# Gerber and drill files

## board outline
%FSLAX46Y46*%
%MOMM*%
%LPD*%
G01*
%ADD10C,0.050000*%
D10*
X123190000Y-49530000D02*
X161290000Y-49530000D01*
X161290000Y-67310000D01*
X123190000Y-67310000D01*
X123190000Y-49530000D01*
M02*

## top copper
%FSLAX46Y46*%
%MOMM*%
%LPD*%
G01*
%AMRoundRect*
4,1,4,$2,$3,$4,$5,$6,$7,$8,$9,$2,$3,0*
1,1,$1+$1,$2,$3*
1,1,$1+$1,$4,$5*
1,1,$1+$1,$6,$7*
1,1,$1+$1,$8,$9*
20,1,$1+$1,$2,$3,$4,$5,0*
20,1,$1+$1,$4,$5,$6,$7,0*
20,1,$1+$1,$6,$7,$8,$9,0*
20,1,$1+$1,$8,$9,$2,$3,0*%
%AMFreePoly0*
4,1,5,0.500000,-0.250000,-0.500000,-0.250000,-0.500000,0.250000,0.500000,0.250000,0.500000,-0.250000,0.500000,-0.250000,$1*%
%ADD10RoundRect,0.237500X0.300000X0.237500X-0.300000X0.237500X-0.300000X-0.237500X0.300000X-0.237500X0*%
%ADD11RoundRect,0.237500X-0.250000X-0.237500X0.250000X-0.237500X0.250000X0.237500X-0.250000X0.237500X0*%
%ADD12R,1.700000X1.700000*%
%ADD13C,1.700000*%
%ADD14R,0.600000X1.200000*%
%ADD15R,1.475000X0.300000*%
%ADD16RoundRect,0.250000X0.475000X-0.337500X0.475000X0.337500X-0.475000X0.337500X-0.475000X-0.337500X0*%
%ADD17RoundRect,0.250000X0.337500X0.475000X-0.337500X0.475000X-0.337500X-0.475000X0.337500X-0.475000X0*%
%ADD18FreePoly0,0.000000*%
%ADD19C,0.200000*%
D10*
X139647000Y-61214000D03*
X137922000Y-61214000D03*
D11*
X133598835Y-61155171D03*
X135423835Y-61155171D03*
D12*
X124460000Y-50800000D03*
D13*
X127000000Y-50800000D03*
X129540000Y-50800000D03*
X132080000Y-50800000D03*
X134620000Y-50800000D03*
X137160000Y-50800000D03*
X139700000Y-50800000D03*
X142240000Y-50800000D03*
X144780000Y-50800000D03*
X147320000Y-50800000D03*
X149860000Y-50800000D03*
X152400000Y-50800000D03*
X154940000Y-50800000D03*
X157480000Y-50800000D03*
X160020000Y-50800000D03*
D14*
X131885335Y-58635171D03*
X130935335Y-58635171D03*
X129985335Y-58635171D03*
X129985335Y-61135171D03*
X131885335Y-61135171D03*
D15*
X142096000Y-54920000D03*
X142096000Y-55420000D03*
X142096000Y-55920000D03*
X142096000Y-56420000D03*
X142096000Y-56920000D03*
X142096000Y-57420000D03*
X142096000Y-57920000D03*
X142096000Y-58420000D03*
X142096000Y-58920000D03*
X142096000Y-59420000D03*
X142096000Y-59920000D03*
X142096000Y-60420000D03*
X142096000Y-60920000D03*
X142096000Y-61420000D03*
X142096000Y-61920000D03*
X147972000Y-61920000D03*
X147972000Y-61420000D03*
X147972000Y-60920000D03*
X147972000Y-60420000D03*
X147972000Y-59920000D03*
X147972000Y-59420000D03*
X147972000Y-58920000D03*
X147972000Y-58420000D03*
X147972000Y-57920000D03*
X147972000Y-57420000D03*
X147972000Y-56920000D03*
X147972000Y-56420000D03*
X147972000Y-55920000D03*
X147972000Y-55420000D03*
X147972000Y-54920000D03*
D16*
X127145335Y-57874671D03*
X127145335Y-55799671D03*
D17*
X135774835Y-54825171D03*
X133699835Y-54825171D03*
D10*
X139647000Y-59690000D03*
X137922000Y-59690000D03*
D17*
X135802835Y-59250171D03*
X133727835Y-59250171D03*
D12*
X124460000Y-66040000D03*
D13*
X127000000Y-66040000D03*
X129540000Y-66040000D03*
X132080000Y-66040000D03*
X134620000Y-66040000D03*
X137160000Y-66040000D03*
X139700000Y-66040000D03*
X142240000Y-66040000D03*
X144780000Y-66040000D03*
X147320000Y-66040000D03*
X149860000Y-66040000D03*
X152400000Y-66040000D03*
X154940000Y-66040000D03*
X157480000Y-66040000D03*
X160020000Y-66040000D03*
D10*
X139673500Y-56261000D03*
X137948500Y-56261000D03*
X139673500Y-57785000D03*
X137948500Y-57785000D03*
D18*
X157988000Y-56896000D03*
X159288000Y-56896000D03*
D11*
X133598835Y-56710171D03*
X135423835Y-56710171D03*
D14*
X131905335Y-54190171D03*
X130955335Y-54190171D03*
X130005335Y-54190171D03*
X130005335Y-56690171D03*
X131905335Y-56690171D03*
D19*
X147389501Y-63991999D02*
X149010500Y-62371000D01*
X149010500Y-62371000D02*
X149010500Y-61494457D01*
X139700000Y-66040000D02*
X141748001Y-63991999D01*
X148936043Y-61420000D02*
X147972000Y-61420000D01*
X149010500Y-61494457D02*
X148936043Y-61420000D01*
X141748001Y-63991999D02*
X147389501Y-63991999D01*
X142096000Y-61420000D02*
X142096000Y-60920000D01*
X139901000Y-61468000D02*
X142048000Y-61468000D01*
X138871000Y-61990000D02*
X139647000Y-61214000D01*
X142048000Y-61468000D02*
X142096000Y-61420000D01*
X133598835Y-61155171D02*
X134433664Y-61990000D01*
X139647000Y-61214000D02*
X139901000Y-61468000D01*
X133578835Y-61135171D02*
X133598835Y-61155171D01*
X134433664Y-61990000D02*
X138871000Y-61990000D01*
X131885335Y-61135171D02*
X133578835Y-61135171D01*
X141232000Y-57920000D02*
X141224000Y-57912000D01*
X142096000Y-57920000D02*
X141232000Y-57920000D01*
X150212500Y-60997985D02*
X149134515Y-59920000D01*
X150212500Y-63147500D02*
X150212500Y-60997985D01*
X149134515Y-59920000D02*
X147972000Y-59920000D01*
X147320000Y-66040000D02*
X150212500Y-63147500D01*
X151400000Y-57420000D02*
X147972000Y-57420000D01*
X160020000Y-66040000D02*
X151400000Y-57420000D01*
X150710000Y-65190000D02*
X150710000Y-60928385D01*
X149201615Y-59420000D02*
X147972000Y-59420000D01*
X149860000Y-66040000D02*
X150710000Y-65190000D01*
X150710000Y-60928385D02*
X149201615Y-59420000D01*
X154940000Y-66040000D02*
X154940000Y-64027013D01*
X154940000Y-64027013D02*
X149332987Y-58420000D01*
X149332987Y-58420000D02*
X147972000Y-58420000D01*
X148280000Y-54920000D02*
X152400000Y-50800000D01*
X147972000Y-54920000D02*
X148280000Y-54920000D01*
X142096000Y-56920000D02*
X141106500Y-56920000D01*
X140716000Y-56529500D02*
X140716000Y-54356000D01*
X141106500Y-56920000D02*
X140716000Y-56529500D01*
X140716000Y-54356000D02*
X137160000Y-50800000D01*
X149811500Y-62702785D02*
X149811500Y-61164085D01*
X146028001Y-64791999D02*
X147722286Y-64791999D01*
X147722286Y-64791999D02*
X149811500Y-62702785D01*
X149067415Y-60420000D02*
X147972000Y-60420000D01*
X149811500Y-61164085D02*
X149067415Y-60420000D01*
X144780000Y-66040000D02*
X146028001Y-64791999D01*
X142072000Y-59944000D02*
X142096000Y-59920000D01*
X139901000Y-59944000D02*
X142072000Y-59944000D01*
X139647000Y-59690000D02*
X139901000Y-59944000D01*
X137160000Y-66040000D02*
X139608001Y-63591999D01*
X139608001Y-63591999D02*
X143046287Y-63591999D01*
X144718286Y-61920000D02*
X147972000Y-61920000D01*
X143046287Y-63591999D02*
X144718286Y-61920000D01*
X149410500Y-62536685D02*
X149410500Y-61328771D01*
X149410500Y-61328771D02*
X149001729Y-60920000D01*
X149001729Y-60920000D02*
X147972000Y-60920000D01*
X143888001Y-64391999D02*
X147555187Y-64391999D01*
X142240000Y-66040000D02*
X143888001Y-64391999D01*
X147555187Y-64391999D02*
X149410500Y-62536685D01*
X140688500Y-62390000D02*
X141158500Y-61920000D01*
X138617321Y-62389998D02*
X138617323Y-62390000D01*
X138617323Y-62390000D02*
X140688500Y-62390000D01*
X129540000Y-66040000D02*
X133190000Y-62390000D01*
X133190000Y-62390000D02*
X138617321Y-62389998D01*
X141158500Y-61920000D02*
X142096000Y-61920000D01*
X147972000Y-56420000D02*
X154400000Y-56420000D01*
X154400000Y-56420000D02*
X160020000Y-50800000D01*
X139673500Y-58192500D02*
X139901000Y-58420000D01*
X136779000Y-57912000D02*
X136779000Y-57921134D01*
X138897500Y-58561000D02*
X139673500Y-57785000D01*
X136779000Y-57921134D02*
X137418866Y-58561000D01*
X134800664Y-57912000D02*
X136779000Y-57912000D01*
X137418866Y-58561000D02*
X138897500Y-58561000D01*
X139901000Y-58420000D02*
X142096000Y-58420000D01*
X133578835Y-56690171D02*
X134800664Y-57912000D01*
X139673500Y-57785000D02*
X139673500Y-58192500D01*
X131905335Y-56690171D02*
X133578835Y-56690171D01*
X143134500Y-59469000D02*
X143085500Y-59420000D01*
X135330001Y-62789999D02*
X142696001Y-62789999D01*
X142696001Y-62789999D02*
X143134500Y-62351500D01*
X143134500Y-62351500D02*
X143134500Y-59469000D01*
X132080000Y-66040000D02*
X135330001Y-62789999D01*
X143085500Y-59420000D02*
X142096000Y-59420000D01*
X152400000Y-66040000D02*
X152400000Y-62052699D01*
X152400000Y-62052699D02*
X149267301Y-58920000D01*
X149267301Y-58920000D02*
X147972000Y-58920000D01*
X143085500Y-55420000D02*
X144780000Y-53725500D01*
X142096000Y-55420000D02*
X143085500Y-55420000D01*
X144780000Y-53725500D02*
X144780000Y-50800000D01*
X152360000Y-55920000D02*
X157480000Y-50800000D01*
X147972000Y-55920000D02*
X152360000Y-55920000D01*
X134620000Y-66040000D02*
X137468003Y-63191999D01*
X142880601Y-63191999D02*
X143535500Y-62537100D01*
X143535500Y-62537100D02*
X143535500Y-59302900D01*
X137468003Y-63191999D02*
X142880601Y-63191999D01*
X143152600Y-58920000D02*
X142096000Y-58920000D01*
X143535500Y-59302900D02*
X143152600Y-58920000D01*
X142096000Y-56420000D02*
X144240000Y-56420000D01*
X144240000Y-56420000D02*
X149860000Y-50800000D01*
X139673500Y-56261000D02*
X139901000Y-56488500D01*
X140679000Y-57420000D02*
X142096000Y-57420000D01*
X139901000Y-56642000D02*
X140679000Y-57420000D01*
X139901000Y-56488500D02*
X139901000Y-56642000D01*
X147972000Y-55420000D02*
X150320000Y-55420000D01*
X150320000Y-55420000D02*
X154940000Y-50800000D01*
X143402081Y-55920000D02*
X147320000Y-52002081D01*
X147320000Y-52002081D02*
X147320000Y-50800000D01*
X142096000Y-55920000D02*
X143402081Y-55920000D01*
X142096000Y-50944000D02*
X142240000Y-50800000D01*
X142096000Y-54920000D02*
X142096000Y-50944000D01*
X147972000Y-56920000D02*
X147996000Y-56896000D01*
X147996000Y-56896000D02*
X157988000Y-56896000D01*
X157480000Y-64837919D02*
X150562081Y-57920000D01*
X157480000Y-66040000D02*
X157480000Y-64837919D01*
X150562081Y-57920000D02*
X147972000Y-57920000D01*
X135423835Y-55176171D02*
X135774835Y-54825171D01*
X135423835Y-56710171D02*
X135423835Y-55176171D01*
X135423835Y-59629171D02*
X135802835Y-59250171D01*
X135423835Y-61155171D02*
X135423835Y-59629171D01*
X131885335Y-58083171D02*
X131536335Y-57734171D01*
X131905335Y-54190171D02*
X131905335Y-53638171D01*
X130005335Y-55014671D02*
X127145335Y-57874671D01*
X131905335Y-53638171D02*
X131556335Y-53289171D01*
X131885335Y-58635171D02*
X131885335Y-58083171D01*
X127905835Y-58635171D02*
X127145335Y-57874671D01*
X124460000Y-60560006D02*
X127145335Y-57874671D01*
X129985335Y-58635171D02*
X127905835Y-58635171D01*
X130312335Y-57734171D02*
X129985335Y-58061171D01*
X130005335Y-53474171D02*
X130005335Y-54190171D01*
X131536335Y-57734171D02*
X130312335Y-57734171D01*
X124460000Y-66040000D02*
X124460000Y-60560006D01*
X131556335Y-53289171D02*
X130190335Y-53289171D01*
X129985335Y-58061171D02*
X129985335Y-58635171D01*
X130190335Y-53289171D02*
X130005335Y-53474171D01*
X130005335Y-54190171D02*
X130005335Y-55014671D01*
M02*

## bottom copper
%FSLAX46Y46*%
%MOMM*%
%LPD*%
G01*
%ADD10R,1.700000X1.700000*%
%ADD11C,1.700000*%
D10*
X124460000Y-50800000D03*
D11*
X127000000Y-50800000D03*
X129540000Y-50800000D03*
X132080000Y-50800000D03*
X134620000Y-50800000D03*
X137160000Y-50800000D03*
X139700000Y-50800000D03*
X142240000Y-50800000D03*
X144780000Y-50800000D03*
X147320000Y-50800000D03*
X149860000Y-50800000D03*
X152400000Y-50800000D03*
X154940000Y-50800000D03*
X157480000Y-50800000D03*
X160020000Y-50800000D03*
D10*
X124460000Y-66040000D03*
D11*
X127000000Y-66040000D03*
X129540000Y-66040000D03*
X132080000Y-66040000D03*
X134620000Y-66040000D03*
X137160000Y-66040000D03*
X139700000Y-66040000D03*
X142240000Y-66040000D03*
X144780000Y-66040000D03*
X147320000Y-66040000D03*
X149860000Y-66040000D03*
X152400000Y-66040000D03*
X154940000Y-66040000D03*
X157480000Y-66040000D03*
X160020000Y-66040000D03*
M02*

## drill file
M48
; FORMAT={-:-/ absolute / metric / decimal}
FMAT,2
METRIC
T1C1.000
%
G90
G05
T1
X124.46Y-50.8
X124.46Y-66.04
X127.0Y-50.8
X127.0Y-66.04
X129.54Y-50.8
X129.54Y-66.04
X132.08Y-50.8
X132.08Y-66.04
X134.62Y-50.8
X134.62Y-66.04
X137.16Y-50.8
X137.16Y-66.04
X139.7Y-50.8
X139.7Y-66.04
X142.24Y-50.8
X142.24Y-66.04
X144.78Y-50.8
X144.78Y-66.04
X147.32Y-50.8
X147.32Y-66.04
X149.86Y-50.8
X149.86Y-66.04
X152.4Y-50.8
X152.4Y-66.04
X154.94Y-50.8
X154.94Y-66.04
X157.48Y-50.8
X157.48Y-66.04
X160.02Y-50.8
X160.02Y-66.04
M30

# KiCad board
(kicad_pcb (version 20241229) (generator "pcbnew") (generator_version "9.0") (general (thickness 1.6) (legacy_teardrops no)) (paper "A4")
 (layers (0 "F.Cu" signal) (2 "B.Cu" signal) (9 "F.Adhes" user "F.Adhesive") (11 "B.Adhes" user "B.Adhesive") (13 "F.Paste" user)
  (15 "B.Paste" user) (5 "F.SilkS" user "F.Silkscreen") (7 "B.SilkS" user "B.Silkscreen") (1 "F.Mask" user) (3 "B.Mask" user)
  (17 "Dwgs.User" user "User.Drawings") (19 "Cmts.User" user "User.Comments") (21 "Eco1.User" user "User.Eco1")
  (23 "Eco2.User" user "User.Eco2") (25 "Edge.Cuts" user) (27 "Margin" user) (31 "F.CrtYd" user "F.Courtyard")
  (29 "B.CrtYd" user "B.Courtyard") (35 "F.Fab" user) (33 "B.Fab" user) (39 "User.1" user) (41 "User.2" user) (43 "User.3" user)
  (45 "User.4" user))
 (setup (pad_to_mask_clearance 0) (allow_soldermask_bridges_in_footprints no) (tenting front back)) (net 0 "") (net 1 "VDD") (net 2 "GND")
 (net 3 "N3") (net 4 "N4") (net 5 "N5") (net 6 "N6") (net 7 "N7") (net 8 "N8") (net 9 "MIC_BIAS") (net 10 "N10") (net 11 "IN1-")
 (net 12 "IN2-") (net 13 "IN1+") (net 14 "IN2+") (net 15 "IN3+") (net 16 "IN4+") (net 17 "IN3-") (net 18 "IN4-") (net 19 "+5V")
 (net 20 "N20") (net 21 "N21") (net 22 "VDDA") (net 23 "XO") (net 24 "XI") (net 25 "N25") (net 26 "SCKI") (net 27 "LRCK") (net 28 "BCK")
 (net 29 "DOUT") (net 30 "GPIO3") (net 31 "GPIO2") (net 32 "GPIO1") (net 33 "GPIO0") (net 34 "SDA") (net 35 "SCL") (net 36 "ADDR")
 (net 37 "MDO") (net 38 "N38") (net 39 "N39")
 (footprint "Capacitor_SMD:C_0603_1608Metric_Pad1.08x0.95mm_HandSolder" (layer "F.Cu") (at 138.7845 61.214 180)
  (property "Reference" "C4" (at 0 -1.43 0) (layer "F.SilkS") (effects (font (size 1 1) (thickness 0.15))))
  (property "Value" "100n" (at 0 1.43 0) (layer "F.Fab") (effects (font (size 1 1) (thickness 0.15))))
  (pad "1" smd roundrect (at -0.8625 0 180) (size 1.075 0.95) (layers "F.Cu" "F.Mask" "F.Paste") (roundrect_rratio 0.25) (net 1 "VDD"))
  (pad "2" smd roundrect (at 0.8625 0 180) (size 1.075 0.95) (layers "F.Cu" "F.Mask" "F.Paste") (roundrect_rratio 0.25) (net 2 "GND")))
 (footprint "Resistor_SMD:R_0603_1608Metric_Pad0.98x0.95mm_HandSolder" (layer "F.Cu") (at 134.511335 61.155171)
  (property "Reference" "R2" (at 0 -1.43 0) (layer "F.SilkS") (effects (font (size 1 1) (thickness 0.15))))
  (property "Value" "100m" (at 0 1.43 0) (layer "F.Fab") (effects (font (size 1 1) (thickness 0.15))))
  (pad "1" smd roundrect (at -0.9125 0) (size 0.975 0.95) (layers "F.Cu" "F.Mask" "F.Paste") (roundrect_rratio 0.25) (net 1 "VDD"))
  (pad "2" smd roundrect (at 0.9125 0) (size 0.975 0.95) (layers "F.Cu" "F.Mask" "F.Paste") (roundrect_rratio 0.25) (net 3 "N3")))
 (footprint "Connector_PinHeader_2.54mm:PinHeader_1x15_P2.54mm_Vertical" (layer "F.Cu") (at 124.46 50.8 90)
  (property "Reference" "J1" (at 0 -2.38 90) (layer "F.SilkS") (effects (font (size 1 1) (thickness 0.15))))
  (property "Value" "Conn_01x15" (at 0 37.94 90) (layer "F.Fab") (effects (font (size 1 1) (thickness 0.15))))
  (pad "1" thru_hole rect (at 0 0 90) (size 1.7 1.7) (drill 1) (layers "*.Cu" "*.Mask") (remove_unused_layers no) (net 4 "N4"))
  (pad "2" thru_hole circle (at 0 2.54 90) (size 1.7 1.7) (drill 1) (layers "*.Cu" "*.Mask") (remove_unused_layers no) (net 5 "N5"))
  (pad "3" thru_hole circle (at 0 5.08 90) (size 1.7 1.7) (drill 1) (layers "*.Cu" "*.Mask") (remove_unused_layers no) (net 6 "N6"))
  (pad "4" thru_hole circle (at 0 7.62 90) (size 1.7 1.7) (drill 1) (layers "*.Cu" "*.Mask") (remove_unused_layers no) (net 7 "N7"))
  (pad "5" thru_hole circle (at 0 10.16 90) (size 1.7 1.7) (drill 1) (layers "*.Cu" "*.Mask") (remove_unused_layers no) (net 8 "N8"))
  (pad "6" thru_hole circle (at 0 12.7 90) (size 1.7 1.7) (drill 1) (layers "*.Cu" "*.Mask") (remove_unused_layers no) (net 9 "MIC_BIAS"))
  (pad "7" thru_hole circle (at 0 15.24 90) (size 1.7 1.7) (drill 1) (layers "*.Cu" "*.Mask") (remove_unused_layers no) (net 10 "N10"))
  (pad "8" thru_hole circle (at 0 17.78 90) (size 1.7 1.7) (drill 1) (layers "*.Cu" "*.Mask") (remove_unused_layers no) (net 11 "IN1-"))
  (pad "9" thru_hole circle (at 0 20.32 90) (size 1.7 1.7) (drill 1) (layers "*.Cu" "*.Mask") (remove_unused_layers no) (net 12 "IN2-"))
  (pad "10" thru_hole circle (at 0 22.86 90) (size 1.7 1.7) (drill 1) (layers "*.Cu" "*.Mask") (remove_unused_layers no) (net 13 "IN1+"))
  (pad "11" thru_hole circle (at 0 25.4 90) (size 1.7 1.7) (drill 1) (layers "*.Cu" "*.Mask") (remove_unused_layers no) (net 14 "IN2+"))
  (pad "12" thru_hole circle (at 0 27.94 90) (size 1.7 1.7) (drill 1) (layers "*.Cu" "*.Mask") (remove_unused_layers no) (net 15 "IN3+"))
  (pad "13" thru_hole circle (at 0 30.48 90) (size 1.7 1.7) (drill 1) (layers "*.Cu" "*.Mask") (remove_unused_layers no) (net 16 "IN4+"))
  (pad "14" thru_hole circle (at 0 33.02 90) (size 1.7 1.7) (drill 1) (layers "*.Cu" "*.Mask") (remove_unused_layers no) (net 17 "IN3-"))
  (pad "15" thru_hole circle (at 0 35.56 90) (size 1.7 1.7) (drill 1) (layers "*.Cu" "*.Mask") (remove_unused_layers no) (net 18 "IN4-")))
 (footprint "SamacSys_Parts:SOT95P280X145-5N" (layer "F.Cu") (at 130.935335 59.885171 -90)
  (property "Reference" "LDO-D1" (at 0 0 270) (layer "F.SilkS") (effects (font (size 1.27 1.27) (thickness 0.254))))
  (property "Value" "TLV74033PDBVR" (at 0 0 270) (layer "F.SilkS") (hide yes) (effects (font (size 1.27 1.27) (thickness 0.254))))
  (pad "1" smd rect (at -1.25 -0.95) (size 0.6 1.2) (layers "F.Cu" "F.Mask" "F.Paste") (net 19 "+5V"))
  (pad "2" smd rect (at -1.25 0) (size 0.6 1.2) (layers "F.Cu" "F.Mask" "F.Paste") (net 2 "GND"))
  (pad "3" smd rect (at -1.25 0.95) (size 0.6 1.2) (layers "F.Cu" "F.Mask" "F.Paste") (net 19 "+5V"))
  (pad "4" smd rect (at 1.25 0.95) (size 0.6 1.2) (layers "F.Cu" "F.Mask" "F.Paste") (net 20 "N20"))
  (pad "5" smd rect (at 1.25 -0.95) (size 0.6 1.2) (layers "F.Cu" "F.Mask" "F.Paste") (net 1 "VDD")))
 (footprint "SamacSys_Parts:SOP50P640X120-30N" (layer "F.Cu") (at 145.034 58.42)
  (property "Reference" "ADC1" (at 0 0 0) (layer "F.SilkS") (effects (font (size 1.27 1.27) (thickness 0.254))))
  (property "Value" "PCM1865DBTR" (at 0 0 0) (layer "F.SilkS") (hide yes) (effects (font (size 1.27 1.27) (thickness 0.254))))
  (pad "1" smd rect (at -2.938 -3.5 90) (size 0.3 1.475) (layers "F.Cu" "F.Mask" "F.Paste") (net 11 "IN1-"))
  (pad "2" smd rect (at -2.938 -3 90) (size 0.3 1.475) (layers "F.Cu" "F.Mask" "F.Paste") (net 12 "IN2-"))
  (pad "3" smd rect (at -2.938 -2.5 90) (size 0.3 1.475) (layers "F.Cu" "F.Mask" "F.Paste") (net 13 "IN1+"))
  (pad "4" smd rect (at -2.938 -2 90) (size 0.3 1.475) (layers "F.Cu" "F.Mask" "F.Paste") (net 14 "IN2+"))
  (pad "5" smd rect (at -2.938 -1.5 90) (size 0.3 1.475) (layers "F.Cu" "F.Mask" "F.Paste") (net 9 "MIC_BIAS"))
  (pad "6" smd rect (at -2.938 -1 90) (size 0.3 1.475) (layers "F.Cu" "F.Mask" "F.Paste") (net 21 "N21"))
  (pad "7" smd rect (at -2.938 -0.5 90) (size 0.3 1.475) (layers "F.Cu" "F.Mask" "F.Paste") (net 2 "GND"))
  (pad "8" smd rect (at -2.938 0 90) (size 0.3 1.475) (layers "F.Cu" "F.Mask" "F.Paste") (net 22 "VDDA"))
  (pad "9" smd rect (at -2.938 0.5 90) (size 0.3 1.475) (layers "F.Cu" "F.Mask" "F.Paste") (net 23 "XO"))
  (pad "10" smd rect (at -2.938 1 90) (size 0.3 1.475) (layers "F.Cu" "F.Mask" "F.Paste") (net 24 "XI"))
  (pad "11" smd rect (at -2.938 1.5 90) (size 0.3 1.475) (layers "F.Cu" "F.Mask" "F.Paste") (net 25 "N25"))
  (pad "12" smd rect (at -2.938 2 90) (size 0.3 1.475) (layers "F.Cu" "F.Mask" "F.Paste") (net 2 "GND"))
  (pad "13" smd rect (at -2.938 2.5 90) (size 0.3 1.475) (layers "F.Cu" "F.Mask" "F.Paste") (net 1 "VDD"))
  (pad "14" smd rect (at -2.938 3 90) (size 0.3 1.475) (layers "F.Cu" "F.Mask" "F.Paste") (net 1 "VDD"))
  (pad "15" smd rect (at -2.938 3.5 90) (size 0.3 1.475) (layers "F.Cu" "F.Mask" "F.Paste") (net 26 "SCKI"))
  (pad "16" smd rect (at 2.938 3.5 90) (size 0.3 1.475) (layers "F.Cu" "F.Mask" "F.Paste") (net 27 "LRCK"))
  (pad "17" smd rect (at 2.938 3 90) (size 0.3 1.475) (layers "F.Cu" "F.Mask" "F.Paste") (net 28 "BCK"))
  (pad "18" smd rect (at 2.938 2.5 90) (size 0.3 1.475) (layers "F.Cu" "F.Mask" "F.Paste") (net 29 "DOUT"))
  (pad "19" smd rect (at 2.938 2 90) (size 0.3 1.475) (layers "F.Cu" "F.Mask" "F.Paste") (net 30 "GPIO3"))
  (pad "20" smd rect (at 2.938 1.5 90) (size 0.3 1.475) (layers "F.Cu" "F.Mask" "F.Paste") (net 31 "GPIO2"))
  (pad "21" smd rect (at 2.938 1 90) (size 0.3 1.475) (layers "F.Cu" "F.Mask" "F.Paste") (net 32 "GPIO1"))
  (pad "22" smd rect (at 2.938 0.5 90) (size 0.3 1.475) (layers "F.Cu" "F.Mask" "F.Paste") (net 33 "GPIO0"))
  (pad "23" smd rect (at 2.938 0 90) (size 0.3 1.475) (layers "F.Cu" "F.Mask" "F.Paste") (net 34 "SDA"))
  (pad "24" smd rect (at 2.938 -0.5 90) (size 0.3 1.475) (layers "F.Cu" "F.Mask" "F.Paste") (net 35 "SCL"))
  (pad "25" smd rect (at 2.938 -1 90) (size 0.3 1.475) (layers "F.Cu" "F.Mask" "F.Paste") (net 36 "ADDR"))
  (pad "26" smd rect (at 2.938 -1.5 90) (size 0.3 1.475) (layers "F.Cu" "F.Mask" "F.Paste") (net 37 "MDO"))
  (pad "27" smd rect (at 2.938 -2 90) (size 0.3 1.475) (layers "F.Cu" "F.Mask" "F.Paste") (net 18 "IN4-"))
  (pad "28" smd rect (at 2.938 -2.5 90) (size 0.3 1.475) (layers "F.Cu" "F.Mask" "F.Paste") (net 17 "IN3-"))
  (pad "29" smd rect (at 2.938 -3 90) (size 0.3 1.475) (layers "F.Cu" "F.Mask" "F.Paste") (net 16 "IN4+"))
  (pad "30" smd rect (at 2.938 -3.5 90) (size 0.3 1.475) (layers "F.Cu" "F.Mask" "F.Paste") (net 15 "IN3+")))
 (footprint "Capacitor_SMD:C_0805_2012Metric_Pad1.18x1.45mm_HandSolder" (layer "F.Cu") (at 127.145335 56.837171 90)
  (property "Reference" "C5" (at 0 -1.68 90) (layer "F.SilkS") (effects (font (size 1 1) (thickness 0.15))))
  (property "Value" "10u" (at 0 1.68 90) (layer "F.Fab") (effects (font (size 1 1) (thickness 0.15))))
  (pad "1" smd roundrect (at -1.0375 0 90) (size 1.175 1.45) (layers "F.Cu" "F.Mask" "F.Paste") (roundrect_rratio 0.212766) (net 19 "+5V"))
  (pad "2" smd roundrect (at 1.0375 0 90) (size 1.175 1.45) (layers "F.Cu" "F.Mask" "F.Paste") (roundrect_rratio 0.212766) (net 2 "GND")))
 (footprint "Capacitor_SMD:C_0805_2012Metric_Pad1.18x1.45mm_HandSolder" (layer "F.Cu") (at 134.737335 54.825171 180)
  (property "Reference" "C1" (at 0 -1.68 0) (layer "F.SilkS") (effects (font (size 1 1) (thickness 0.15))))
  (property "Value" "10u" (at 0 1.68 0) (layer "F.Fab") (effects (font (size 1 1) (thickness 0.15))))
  (pad "1" smd roundrect (at -1.0375 0 180) (size 1.175 1.45) (layers "F.Cu" "F.Mask" "F.Paste") (roundrect_rratio 0.212766) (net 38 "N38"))
  (pad "2" smd roundrect (at 1.0375 0 180) (size 1.175 1.45) (layers "F.Cu" "F.Mask" "F.Paste") (roundrect_rratio 0.212766) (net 2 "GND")))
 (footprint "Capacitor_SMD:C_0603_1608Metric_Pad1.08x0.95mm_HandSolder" (layer "F.Cu") (at 138.7845 59.69 180)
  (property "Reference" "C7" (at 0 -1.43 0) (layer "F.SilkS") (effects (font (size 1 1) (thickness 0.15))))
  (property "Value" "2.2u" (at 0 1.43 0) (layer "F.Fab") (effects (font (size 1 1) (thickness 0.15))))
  (pad "1" smd roundrect (at -0.8625 0 180) (size 1.075 0.95) (layers "F.Cu" "F.Mask" "F.Paste") (roundrect_rratio 0.25) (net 25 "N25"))
  (pad "2" smd roundrect (at 0.8625 0 180) (size 1.075 0.95) (layers "F.Cu" "F.Mask" "F.Paste") (roundrect_rratio 0.25) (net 2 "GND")))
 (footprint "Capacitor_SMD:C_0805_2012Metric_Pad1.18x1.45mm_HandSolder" (layer "F.Cu") (at 134.765335 59.250171 180)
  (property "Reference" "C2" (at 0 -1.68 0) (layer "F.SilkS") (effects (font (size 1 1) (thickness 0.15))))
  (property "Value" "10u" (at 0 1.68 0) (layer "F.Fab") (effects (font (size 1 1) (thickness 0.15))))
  (pad "1" smd roundrect (at -1.0375 0 180) (size 1.175 1.45) (layers "F.Cu" "F.Mask" "F.Paste") (roundrect_rratio 0.212766) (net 3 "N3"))
  (pad "2" smd roundrect (at 1.0375 0 180) (size 1.175 1.45) (layers "F.Cu" "F.Mask" "F.Paste") (roundrect_rratio 0.212766) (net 2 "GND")))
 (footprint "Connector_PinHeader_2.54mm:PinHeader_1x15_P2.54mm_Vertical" (layer "F.Cu") (at 124.46 66.04 90)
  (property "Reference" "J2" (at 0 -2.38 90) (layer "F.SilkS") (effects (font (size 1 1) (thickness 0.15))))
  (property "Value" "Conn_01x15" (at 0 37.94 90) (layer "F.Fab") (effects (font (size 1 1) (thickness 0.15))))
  (pad "1" thru_hole rect (at 0 0 90) (size 1.7 1.7) (drill 1) (layers "*.Cu" "*.Mask") (remove_unused_layers no) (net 19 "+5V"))
  (pad "2" thru_hole circle (at 0 2.54 90) (size 1.7 1.7) (drill 1) (layers "*.Cu" "*.Mask") (remove_unused_layers no) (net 2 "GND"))
  (pad "3" thru_hole circle (at 0 5.08 90) (size 1.7 1.7) (drill 1) (layers "*.Cu" "*.Mask") (remove_unused_layers no) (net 26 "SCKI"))
  (pad "4" thru_hole circle (at 0 7.62 90) (size 1.7 1.7) (drill 1) (layers "*.Cu" "*.Mask") (remove_unused_layers no) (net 24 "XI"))
  (pad "5" thru_hole circle (at 0 10.16 90) (size 1.7 1.7) (drill 1) (layers "*.Cu" "*.Mask") (remove_unused_layers no) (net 23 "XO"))
  (pad "6" thru_hole circle (at 0 12.7 90) (size 1.7 1.7) (drill 1) (layers "*.Cu" "*.Mask") (remove_unused_layers no) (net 27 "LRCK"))
  (pad "7" thru_hole circle (at 0 15.24 90) (size 1.7 1.7) (drill 1) (layers "*.Cu" "*.Mask") (remove_unused_layers no) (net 28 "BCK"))
  (pad "8" thru_hole circle (at 0 17.78 90) (size 1.7 1.7) (drill 1) (layers "*.Cu" "*.Mask") (remove_unused_layers no) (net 29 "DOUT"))
  (pad "9" thru_hole circle (at 0 20.32 90) (size 1.7 1.7) (drill 1) (layers "*.Cu" "*.Mask") (remove_unused_layers no) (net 30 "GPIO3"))
  (pad "10" thru_hole circle (at 0 22.86 90) (size 1.7 1.7) (drill 1) (layers "*.Cu" "*.Mask") (remove_unused_layers no) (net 31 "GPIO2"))
  (pad "11" thru_hole circle (at 0 25.4 90) (size 1.7 1.7) (drill 1) (layers "*.Cu" "*.Mask") (remove_unused_layers no) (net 32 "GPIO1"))
  (pad "12" thru_hole circle (at 0 27.94 90) (size 1.7 1.7) (drill 1) (layers "*.Cu" "*.Mask") (remove_unused_layers no) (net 33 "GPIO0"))
  (pad "13" thru_hole circle (at 0 30.48 90) (size 1.7 1.7) (drill 1) (layers "*.Cu" "*.Mask") (remove_unused_layers no) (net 34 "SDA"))
  (pad "14" thru_hole circle (at 0 33.02 90) (size 1.7 1.7) (drill 1) (layers "*.Cu" "*.Mask") (remove_unused_layers no) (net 35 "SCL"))
  (pad "15" thru_hole circle (at 0 35.56 90) (size 1.7 1.7) (drill 1) (layers "*.Cu" "*.Mask") (remove_unused_layers no) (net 36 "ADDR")))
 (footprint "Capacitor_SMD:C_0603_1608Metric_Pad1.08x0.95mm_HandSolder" (layer "F.Cu") (at 138.811 56.261 180)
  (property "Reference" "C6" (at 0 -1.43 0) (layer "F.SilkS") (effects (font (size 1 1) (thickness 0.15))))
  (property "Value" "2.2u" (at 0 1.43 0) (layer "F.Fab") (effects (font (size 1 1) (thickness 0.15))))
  (pad "1" smd roundrect (at -0.8625 0 180) (size 1.075 0.95) (layers "F.Cu" "F.Mask" "F.Paste") (roundrect_rratio 0.25) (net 21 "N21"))
  (pad "2" smd roundrect (at 0.8625 0 180) (size 1.075 0.95) (layers "F.Cu" "F.Mask" "F.Paste") (roundrect_rratio 0.25) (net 2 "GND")))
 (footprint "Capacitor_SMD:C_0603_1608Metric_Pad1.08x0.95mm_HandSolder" (layer "F.Cu") (at 138.811 57.785 180)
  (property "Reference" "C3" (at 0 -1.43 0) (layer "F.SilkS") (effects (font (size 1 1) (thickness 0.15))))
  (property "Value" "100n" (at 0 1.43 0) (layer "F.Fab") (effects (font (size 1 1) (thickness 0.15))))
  (pad "1" smd roundrect (at -0.8625 0 180) (size 1.075 0.95) (layers "F.Cu" "F.Mask" "F.Paste") (roundrect_rratio 0.25) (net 22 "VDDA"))
  (pad "2" smd roundrect (at 0.8625 0 180) (size 1.075 0.95) (layers "F.Cu" "F.Mask" "F.Paste") (roundrect_rratio 0.25) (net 2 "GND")))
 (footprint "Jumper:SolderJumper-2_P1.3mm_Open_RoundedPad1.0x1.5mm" (layer "F.Cu") (at 158.638 56.896)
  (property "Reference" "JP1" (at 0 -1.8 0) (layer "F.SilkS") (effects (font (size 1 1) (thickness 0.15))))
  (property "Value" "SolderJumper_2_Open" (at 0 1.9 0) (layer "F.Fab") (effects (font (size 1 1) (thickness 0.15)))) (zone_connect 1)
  (pad "1" smd custom (at -0.65 0) (size 1 0.5) (layers "F.Cu" "F.Mask") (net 37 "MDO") (zone_connect 2) (thermal_bridge_angle 45)
   (options (clearance outline) (anchor rect)) (primitives))
  (pad "2" smd custom (at 0.65 0) (size 1 0.5) (layers "F.Cu" "F.Mask") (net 1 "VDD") (zone_connect 2) (thermal_bridge_angle 45)
   (options (clearance outline) (anchor rect)) (primitives)))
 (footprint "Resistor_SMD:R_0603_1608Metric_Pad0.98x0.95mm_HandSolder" (layer "F.Cu") (at 134.511335 56.710171)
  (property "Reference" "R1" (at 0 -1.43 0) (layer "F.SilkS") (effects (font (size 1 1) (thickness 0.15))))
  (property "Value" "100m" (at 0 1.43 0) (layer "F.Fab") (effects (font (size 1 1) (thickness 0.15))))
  (pad "1" smd roundrect (at -0.9125 0) (size 0.975 0.95) (layers "F.Cu" "F.Mask" "F.Paste") (roundrect_rratio 0.25) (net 22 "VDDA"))
  (pad "2" smd roundrect (at 0.9125 0) (size 0.975 0.95) (layers "F.Cu" "F.Mask" "F.Paste") (roundrect_rratio 0.25) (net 38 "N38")))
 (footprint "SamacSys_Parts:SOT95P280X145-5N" (layer "F.Cu") (at 130.955335 55.440171 -90)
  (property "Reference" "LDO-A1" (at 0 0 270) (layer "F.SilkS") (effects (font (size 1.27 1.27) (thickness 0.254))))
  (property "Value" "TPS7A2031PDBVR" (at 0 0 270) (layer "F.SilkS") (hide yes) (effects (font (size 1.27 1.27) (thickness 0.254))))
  (pad "1" smd rect (at -1.25 -0.95) (size 0.6 1.2) (layers "F.Cu" "F.Mask" "F.Paste") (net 19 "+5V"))
  (pad "2" smd rect (at -1.25 0) (size 0.6 1.2) (layers "F.Cu" "F.Mask" "F.Paste") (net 2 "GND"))
  (pad "3" smd rect (at -1.25 0.95) (size 0.6 1.2) (layers "F.Cu" "F.Mask" "F.Paste") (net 19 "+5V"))
  (pad "4" smd rect (at 1.25 0.95) (size 0.6 1.2) (layers "F.Cu" "F.Mask" "F.Paste") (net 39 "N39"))
  (pad "5" smd rect (at 1.25 -0.95) (size 0.6 1.2) (layers "F.Cu" "F.Mask" "F.Paste") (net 22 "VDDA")))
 (gr_rect (start 123.19 49.53) (end 161.29 67.31) (stroke (width 0.05) (type default)) (fill no) (layer "Edge.Cuts"))
 (segment (start 147.389501 63.991999) (end 149.0105 62.371) (width 0.2) (layer "F.Cu") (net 28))
 (segment (start 149.0105 62.371) (end 149.0105 61.494457) (width 0.2) (layer "F.Cu") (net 28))
 (segment (start 139.7 66.04) (end 141.748001 63.991999) (width 0.2) (layer "F.Cu") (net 28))
 (segment (start 148.936043 61.42) (end 147.972 61.42) (width 0.2) (layer "F.Cu") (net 28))
 (segment (start 149.0105 61.494457) (end 148.936043 61.42) (width 0.2) (layer "F.Cu") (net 28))
 (segment (start 141.748001 63.991999) (end 147.389501 63.991999) (width 0.2) (layer "F.Cu") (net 28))
 (segment (start 142.096 61.42) (end 142.096 60.92) (width 0.2) (layer "F.Cu") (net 1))
 (segment (start 139.901 61.468) (end 142.048 61.468) (width 0.2) (layer "F.Cu") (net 1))
 (segment (start 138.871 61.99) (end 139.647 61.214) (width 0.2) (layer "F.Cu") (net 1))
 (segment (start 142.048 61.468) (end 142.096 61.42) (width 0.2) (layer "F.Cu") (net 1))
 (segment (start 133.598835 61.155171) (end 134.433664 61.99) (width 0.2) (layer "F.Cu") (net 1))
 (segment (start 139.647 61.214) (end 139.901 61.468) (width 0.2) (layer "F.Cu") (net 1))
 (segment (start 133.578835 61.135171) (end 133.598835 61.155171) (width 0.2) (layer "F.Cu") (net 1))
 (segment (start 134.433664 61.99) (end 138.871 61.99) (width 0.2) (layer "F.Cu") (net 1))
 (segment (start 131.885335 61.135171) (end 133.578835 61.135171) (width 0.2) (layer "F.Cu") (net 1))
 (segment (start 141.232 57.92) (end 141.224 57.912) (width 0.2) (layer "F.Cu") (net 2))
 (segment (start 142.096 57.92) (end 141.232 57.92) (width 0.2) (layer "F.Cu") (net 2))
 (segment (start 150.2125 60.997985) (end 149.134515 59.92) (width 0.2) (layer "F.Cu") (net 31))
 (segment (start 150.2125 63.1475) (end 150.2125 60.997985) (width 0.2) (layer "F.Cu") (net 31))
 (segment (start 149.134515 59.92) (end 147.972 59.92) (width 0.2) (layer "F.Cu") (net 31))
 (segment (start 147.32 66.04) (end 150.2125 63.1475) (width 0.2) (layer "F.Cu") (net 31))
 (segment (start 151.4 57.42) (end 147.972 57.42) (width 0.2) (layer "F.Cu") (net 36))
 (segment (start 160.02 66.04) (end 151.4 57.42) (width 0.2) (layer "F.Cu") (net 36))
 (segment (start 150.71 65.19) (end 150.71 60.928385) (width 0.2) (layer "F.Cu") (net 32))
 (segment (start 149.201615 59.42) (end 147.972 59.42) (width 0.2) (layer "F.Cu") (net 32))
 (segment (start 149.86 66.04) (end 150.71 65.19) (width 0.2) (layer "F.Cu") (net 32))
 (segment (start 150.71 60.928385) (end 149.201615 59.42) (width 0.2) (layer "F.Cu") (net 32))
 (segment (start 154.94 66.04) (end 154.94 64.027013) (width 0.2) (layer "F.Cu") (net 34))
 (segment (start 154.94 64.027013) (end 149.332987 58.42) (width 0.2) (layer "F.Cu") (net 34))
 (segment (start 149.332987 58.42) (end 147.972 58.42) (width 0.2) (layer "F.Cu") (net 34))
 (segment (start 148.28 54.92) (end 152.4 50.8) (width 0.2) (layer "F.Cu") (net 15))
 (segment (start 147.972 54.92) (end 148.28 54.92) (width 0.2) (layer "F.Cu") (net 15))
 (segment (start 142.096 56.92) (end 141.1065 56.92) (width 0.2) (layer "F.Cu") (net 9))
 (segment (start 140.716 56.5295) (end 140.716 54.356) (width 0.2) (layer "F.Cu") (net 9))
 (segment (start 141.1065 56.92) (end 140.716 56.5295) (width 0.2) (layer "F.Cu") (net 9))
 (segment (start 140.716 54.356) (end 137.16 50.8) (width 0.2) (layer "F.Cu") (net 9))
 (segment (start 149.8115 62.702785) (end 149.8115 61.164085) (width 0.2) (layer "F.Cu") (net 30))
 (segment (start 146.028001 64.791999) (end 147.722286 64.791999) (width 0.2) (layer "F.Cu") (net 30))
 (segment (start 147.722286 64.791999) (end 149.8115 62.702785) (width 0.2) (layer "F.Cu") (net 30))
 (segment (start 149.067415 60.42) (end 147.972 60.42) (width 0.2) (layer "F.Cu") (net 30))
 (segment (start 149.8115 61.164085) (end 149.067415 60.42) (width 0.2) (layer "F.Cu") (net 30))
 (segment (start 144.78 66.04) (end 146.028001 64.791999) (width 0.2) (layer "F.Cu") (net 30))
 (segment (start 142.072 59.944) (end 142.096 59.92) (width 0.2) (layer "F.Cu") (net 25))
 (segment (start 139.901 59.944) (end 142.072 59.944) (width 0.2) (layer "F.Cu") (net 25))
 (segment (start 139.647 59.69) (end 139.901 59.944) (width 0.2) (layer "F.Cu") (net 25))
 (segment (start 137.16 66.04) (end 139.608001 63.591999) (width 0.2) (layer "F.Cu") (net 27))
 (segment (start 139.608001 63.591999) (end 143.046287 63.591999) (width 0.2) (layer "F.Cu") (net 27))
 (segment (start 144.718286 61.92) (end 147.972 61.92) (width 0.2) (layer "F.Cu") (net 27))
 (segment (start 143.046287 63.591999) (end 144.718286 61.92) (width 0.2) (layer "F.Cu") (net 27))
 (segment (start 149.4105 62.536685) (end 149.4105 61.328771) (width 0.2) (layer "F.Cu") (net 29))
 (segment (start 149.4105 61.328771) (end 149.001729 60.92) (width 0.2) (layer "F.Cu") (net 29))
 (segment (start 149.001729 60.92) (end 147.972 60.92) (width 0.2) (layer "F.Cu") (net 29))
 (segment (start 143.888001 64.391999) (end 147.555187 64.391999) (width 0.2) (layer "F.Cu") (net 29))
 (segment (start 142.24 66.04) (end 143.888001 64.391999) (width 0.2) (layer "F.Cu") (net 29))
 (segment (start 147.555187 64.391999) (end 149.4105 62.536685) (width 0.2) (layer "F.Cu") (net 29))
 (segment (start 140.6885 62.39) (end 141.1585 61.92) (width 0.2) (layer "F.Cu") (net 26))
 (segment (start 138.617321 62.389998) (end 138.617323 62.39) (width 0.2) (layer "F.Cu") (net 26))
 (segment (start 138.617323 62.39) (end 140.6885 62.39) (width 0.2) (layer "F.Cu") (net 26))
 (segment (start 129.54 66.04) (end 133.19 62.39) (width 0.2) (layer "F.Cu") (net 26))
 (segment (start 133.19 62.39) (end 138.617321 62.389998) (width 0.2) (layer "F.Cu") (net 26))
 (segment (start 141.1585 61.92) (end 142.096 61.92) (width 0.2) (layer "F.Cu") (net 26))
 (segment (start 147.972 56.42) (end 154.4 56.42) (width 0.2) (layer "F.Cu") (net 18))
 (segment (start 154.4 56.42) (end 160.02 50.8) (width 0.2) (layer "F.Cu") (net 18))
 (segment (start 139.6735 58.1925) (end 139.901 58.42) (width 0.2) (layer "F.Cu") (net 22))
 (segment (start 136.779 57.912) (end 136.779 57.921134) (width 0.2) (layer "F.Cu") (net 22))
 (segment (start 138.8975 58.561) (end 139.6735 57.785) (width 0.2) (layer "F.Cu") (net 22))
 (segment (start 136.779 57.921134) (end 137.418866 58.561) (width 0.2) (layer "F.Cu") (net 22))
 (segment (start 134.800664 57.912) (end 136.779 57.912) (width 0.2) (layer "F.Cu") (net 22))
 (segment (start 137.418866 58.561) (end 138.8975 58.561) (width 0.2) (layer "F.Cu") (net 22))
 (segment (start 139.901 58.42) (end 142.096 58.42) (width 0.2) (layer "F.Cu") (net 22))
 (segment (start 133.578835 56.690171) (end 134.800664 57.912) (width 0.2) (layer "F.Cu") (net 22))
 (segment (start 139.6735 57.785) (end 139.6735 58.1925) (width 0.2) (layer "F.Cu") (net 22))
 (segment (start 131.905335 56.690171) (end 133.578835 56.690171) (width 0.2) (layer "F.Cu") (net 22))
 (segment (start 143.1345 59.469) (end 143.0855 59.42) (width 0.2) (layer "F.Cu") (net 24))
 (segment (start 135.330001 62.789999) (end 142.696001 62.789999) (width 0.2) (layer "F.Cu") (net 24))
 (segment (start 142.696001 62.789999) (end 143.1345 62.3515) (width 0.2) (layer "F.Cu") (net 24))
 (segment (start 143.1345 62.3515) (end 143.1345 59.469) (width 0.2) (layer "F.Cu") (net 24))
 (segment (start 132.08 66.04) (end 135.330001 62.789999) (width 0.2) (layer "F.Cu") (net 24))
 (segment (start 143.0855 59.42) (end 142.096 59.42) (width 0.2) (layer "F.Cu") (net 24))
 (segment (start 152.4 66.04) (end 152.4 62.052699) (width 0.2) (layer "F.Cu") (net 33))
 (segment (start 152.4 62.052699) (end 149.267301 58.92) (width 0.2) (layer "F.Cu") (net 33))
 (segment (start 149.267301 58.92) (end 147.972 58.92) (width 0.2) (layer "F.Cu") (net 33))
 (segment (start 143.0855 55.42) (end 144.78 53.7255) (width 0.2) (layer "F.Cu") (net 12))
 (segment (start 142.096 55.42) (end 143.0855 55.42) (width 0.2) (layer "F.Cu") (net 12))
 (segment (start 144.78 53.7255) (end 144.78 50.8) (width 0.2) (layer "F.Cu") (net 12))
 (segment (start 152.36 55.92) (end 157.48 50.8) (width 0.2) (layer "F.Cu") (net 17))
 (segment (start 147.972 55.92) (end 152.36 55.92) (width 0.2) (layer "F.Cu") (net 17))
 (segment (start 134.62 66.04) (end 137.468003 63.191999) (width 0.2) (layer "F.Cu") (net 23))
 (segment (start 142.880601 63.191999) (end 143.5355 62.5371) (width 0.2) (layer "F.Cu") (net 23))
 (segment (start 143.5355 62.5371) (end 143.5355 59.3029) (width 0.2) (layer "F.Cu") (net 23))
 (segment (start 137.468003 63.191999) (end 142.880601 63.191999) (width 0.2) (layer "F.Cu") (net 23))
 (segment (start 143.1526 58.92) (end 142.096 58.92) (width 0.2) (layer "F.Cu") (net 23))
 (segment (start 143.5355 59.3029) (end 143.1526 58.92) (width 0.2) (layer "F.Cu") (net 23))
 (segment (start 142.096 56.42) (end 144.24 56.42) (width 0.2) (layer "F.Cu") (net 14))
 (segment (start 144.24 56.42) (end 149.86 50.8) (width 0.2) (layer "F.Cu") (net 14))
 (segment (start 139.6735 56.261) (end 139.901 56.4885) (width 0.2) (layer "F.Cu") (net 21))
 (segment (start 140.679 57.42) (end 142.096 57.42) (width 0.2) (layer "F.Cu") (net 21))
 (segment (start 139.901 56.642) (end 140.679 57.42) (width 0.2) (layer "F.Cu") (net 21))
 (segment (start 139.901 56.4885) (end 139.901 56.642) (width 0.2) (layer "F.Cu") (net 21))
 (segment (start 147.972 55.42) (end 150.32 55.42) (width 0.2) (layer "F.Cu") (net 16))
 (segment (start 150.32 55.42) (end 154.94 50.8) (width 0.2) (layer "F.Cu") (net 16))
 (segment (start 143.402081 55.92) (end 147.32 52.002081) (width 0.2) (layer "F.Cu") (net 13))
 (segment (start 147.32 52.002081) (end 147.32 50.8) (width 0.2) (layer "F.Cu") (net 13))
 (segment (start 142.096 55.92) (end 143.402081 55.92) (width 0.2) (layer "F.Cu") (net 13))
 (segment (start 142.096 50.944) (end 142.24 50.8) (width 0.2) (layer "F.Cu") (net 11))
 (segment (start 142.096 54.92) (end 142.096 50.944) (width 0.2) (layer "F.Cu") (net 11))
 (segment (start 147.972 56.92) (end 147.996 56.896) (width 0.2) (layer "F.Cu") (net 37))
 (segment (start 147.996 56.896) (end 157.988 56.896) (width 0.2) (layer "F.Cu") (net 37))
 (segment (start 157.48 64.837919) (end 150.562081 57.92) (width 0.2) (layer "F.Cu") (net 35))
 (segment (start 157.48 66.04) (end 157.48 64.837919) (width 0.2) (layer "F.Cu") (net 35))
 (segment (start 150.562081 57.92) (end 147.972 57.92) (width 0.2) (layer "F.Cu") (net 35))
 (segment (start 135.423835 55.176171) (end 135.774835 54.825171) (width 0.2) (layer "F.Cu") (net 38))
 (segment (start 135.423835 56.710171) (end 135.423835 55.176171) (width 0.2) (layer "F.Cu") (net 38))
 (segment (start 135.423835 59.629171) (end 135.802835 59.250171) (width 0.2) (layer "F.Cu") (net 3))
 (segment (start 135.423835 61.155171) (end 135.423835 59.629171) (width 0.2) (layer "F.Cu") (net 3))
 (segment (start 131.885335 58.083171) (end 131.536335 57.734171) (width 0.2) (layer "F.Cu") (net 19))
 (segment (start 131.905335 54.190171) (end 131.905335 53.638171) (width 0.2) (layer "F.Cu") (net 19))
 (segment (start 130.005335 55.014671) (end 127.145335 57.874671) (width 0.2) (layer "F.Cu") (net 19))
 (segment (start 131.905335 53.638171) (end 131.556335 53.289171) (width 0.2) (layer "F.Cu") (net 19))
 (segment (start 131.885335 58.635171) (end 131.885335 58.083171) (width 0.2) (layer "F.Cu") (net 19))
 (segment (start 127.905835 58.635171) (end 127.145335 57.874671) (width 0.2) (layer "F.Cu") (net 19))
 (segment (start 124.46 60.560006) (end 127.145335 57.874671) (width 0.2) (layer "F.Cu") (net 19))
 (segment (start 129.985335 58.635171) (end 127.905835 58.635171) (width 0.2) (layer "F.Cu") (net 19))
 (segment (start 130.312335 57.734171) (end 129.985335 58.061171) (width 0.2) (layer "F.Cu") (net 19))
 (segment (start 130.005335 53.474171) (end 130.005335 54.190171) (width 0.2) (layer "F.Cu") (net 19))
 (segment (start 131.536335 57.734171) (end 130.312335 57.734171) (width 0.2) (layer "F.Cu") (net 19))
 (segment (start 124.46 66.04) (end 124.46 60.560006) (width 0.2) (layer "F.Cu") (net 19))
 (segment (start 131.556335 53.289171) (end 130.190335 53.289171) (width 0.2) (layer "F.Cu") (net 19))
 (segment (start 129.985335 58.061171) (end 129.985335 58.635171) (width 0.2) (layer "F.Cu") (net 19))
 (segment (start 130.190335 53.289171) (end 130.005335 53.474171) (width 0.2) (layer "F.Cu") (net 19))
 (segment (start 130.005335 54.190171) (end 130.005335 55.014671) (width 0.2) (layer "F.Cu") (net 19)))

